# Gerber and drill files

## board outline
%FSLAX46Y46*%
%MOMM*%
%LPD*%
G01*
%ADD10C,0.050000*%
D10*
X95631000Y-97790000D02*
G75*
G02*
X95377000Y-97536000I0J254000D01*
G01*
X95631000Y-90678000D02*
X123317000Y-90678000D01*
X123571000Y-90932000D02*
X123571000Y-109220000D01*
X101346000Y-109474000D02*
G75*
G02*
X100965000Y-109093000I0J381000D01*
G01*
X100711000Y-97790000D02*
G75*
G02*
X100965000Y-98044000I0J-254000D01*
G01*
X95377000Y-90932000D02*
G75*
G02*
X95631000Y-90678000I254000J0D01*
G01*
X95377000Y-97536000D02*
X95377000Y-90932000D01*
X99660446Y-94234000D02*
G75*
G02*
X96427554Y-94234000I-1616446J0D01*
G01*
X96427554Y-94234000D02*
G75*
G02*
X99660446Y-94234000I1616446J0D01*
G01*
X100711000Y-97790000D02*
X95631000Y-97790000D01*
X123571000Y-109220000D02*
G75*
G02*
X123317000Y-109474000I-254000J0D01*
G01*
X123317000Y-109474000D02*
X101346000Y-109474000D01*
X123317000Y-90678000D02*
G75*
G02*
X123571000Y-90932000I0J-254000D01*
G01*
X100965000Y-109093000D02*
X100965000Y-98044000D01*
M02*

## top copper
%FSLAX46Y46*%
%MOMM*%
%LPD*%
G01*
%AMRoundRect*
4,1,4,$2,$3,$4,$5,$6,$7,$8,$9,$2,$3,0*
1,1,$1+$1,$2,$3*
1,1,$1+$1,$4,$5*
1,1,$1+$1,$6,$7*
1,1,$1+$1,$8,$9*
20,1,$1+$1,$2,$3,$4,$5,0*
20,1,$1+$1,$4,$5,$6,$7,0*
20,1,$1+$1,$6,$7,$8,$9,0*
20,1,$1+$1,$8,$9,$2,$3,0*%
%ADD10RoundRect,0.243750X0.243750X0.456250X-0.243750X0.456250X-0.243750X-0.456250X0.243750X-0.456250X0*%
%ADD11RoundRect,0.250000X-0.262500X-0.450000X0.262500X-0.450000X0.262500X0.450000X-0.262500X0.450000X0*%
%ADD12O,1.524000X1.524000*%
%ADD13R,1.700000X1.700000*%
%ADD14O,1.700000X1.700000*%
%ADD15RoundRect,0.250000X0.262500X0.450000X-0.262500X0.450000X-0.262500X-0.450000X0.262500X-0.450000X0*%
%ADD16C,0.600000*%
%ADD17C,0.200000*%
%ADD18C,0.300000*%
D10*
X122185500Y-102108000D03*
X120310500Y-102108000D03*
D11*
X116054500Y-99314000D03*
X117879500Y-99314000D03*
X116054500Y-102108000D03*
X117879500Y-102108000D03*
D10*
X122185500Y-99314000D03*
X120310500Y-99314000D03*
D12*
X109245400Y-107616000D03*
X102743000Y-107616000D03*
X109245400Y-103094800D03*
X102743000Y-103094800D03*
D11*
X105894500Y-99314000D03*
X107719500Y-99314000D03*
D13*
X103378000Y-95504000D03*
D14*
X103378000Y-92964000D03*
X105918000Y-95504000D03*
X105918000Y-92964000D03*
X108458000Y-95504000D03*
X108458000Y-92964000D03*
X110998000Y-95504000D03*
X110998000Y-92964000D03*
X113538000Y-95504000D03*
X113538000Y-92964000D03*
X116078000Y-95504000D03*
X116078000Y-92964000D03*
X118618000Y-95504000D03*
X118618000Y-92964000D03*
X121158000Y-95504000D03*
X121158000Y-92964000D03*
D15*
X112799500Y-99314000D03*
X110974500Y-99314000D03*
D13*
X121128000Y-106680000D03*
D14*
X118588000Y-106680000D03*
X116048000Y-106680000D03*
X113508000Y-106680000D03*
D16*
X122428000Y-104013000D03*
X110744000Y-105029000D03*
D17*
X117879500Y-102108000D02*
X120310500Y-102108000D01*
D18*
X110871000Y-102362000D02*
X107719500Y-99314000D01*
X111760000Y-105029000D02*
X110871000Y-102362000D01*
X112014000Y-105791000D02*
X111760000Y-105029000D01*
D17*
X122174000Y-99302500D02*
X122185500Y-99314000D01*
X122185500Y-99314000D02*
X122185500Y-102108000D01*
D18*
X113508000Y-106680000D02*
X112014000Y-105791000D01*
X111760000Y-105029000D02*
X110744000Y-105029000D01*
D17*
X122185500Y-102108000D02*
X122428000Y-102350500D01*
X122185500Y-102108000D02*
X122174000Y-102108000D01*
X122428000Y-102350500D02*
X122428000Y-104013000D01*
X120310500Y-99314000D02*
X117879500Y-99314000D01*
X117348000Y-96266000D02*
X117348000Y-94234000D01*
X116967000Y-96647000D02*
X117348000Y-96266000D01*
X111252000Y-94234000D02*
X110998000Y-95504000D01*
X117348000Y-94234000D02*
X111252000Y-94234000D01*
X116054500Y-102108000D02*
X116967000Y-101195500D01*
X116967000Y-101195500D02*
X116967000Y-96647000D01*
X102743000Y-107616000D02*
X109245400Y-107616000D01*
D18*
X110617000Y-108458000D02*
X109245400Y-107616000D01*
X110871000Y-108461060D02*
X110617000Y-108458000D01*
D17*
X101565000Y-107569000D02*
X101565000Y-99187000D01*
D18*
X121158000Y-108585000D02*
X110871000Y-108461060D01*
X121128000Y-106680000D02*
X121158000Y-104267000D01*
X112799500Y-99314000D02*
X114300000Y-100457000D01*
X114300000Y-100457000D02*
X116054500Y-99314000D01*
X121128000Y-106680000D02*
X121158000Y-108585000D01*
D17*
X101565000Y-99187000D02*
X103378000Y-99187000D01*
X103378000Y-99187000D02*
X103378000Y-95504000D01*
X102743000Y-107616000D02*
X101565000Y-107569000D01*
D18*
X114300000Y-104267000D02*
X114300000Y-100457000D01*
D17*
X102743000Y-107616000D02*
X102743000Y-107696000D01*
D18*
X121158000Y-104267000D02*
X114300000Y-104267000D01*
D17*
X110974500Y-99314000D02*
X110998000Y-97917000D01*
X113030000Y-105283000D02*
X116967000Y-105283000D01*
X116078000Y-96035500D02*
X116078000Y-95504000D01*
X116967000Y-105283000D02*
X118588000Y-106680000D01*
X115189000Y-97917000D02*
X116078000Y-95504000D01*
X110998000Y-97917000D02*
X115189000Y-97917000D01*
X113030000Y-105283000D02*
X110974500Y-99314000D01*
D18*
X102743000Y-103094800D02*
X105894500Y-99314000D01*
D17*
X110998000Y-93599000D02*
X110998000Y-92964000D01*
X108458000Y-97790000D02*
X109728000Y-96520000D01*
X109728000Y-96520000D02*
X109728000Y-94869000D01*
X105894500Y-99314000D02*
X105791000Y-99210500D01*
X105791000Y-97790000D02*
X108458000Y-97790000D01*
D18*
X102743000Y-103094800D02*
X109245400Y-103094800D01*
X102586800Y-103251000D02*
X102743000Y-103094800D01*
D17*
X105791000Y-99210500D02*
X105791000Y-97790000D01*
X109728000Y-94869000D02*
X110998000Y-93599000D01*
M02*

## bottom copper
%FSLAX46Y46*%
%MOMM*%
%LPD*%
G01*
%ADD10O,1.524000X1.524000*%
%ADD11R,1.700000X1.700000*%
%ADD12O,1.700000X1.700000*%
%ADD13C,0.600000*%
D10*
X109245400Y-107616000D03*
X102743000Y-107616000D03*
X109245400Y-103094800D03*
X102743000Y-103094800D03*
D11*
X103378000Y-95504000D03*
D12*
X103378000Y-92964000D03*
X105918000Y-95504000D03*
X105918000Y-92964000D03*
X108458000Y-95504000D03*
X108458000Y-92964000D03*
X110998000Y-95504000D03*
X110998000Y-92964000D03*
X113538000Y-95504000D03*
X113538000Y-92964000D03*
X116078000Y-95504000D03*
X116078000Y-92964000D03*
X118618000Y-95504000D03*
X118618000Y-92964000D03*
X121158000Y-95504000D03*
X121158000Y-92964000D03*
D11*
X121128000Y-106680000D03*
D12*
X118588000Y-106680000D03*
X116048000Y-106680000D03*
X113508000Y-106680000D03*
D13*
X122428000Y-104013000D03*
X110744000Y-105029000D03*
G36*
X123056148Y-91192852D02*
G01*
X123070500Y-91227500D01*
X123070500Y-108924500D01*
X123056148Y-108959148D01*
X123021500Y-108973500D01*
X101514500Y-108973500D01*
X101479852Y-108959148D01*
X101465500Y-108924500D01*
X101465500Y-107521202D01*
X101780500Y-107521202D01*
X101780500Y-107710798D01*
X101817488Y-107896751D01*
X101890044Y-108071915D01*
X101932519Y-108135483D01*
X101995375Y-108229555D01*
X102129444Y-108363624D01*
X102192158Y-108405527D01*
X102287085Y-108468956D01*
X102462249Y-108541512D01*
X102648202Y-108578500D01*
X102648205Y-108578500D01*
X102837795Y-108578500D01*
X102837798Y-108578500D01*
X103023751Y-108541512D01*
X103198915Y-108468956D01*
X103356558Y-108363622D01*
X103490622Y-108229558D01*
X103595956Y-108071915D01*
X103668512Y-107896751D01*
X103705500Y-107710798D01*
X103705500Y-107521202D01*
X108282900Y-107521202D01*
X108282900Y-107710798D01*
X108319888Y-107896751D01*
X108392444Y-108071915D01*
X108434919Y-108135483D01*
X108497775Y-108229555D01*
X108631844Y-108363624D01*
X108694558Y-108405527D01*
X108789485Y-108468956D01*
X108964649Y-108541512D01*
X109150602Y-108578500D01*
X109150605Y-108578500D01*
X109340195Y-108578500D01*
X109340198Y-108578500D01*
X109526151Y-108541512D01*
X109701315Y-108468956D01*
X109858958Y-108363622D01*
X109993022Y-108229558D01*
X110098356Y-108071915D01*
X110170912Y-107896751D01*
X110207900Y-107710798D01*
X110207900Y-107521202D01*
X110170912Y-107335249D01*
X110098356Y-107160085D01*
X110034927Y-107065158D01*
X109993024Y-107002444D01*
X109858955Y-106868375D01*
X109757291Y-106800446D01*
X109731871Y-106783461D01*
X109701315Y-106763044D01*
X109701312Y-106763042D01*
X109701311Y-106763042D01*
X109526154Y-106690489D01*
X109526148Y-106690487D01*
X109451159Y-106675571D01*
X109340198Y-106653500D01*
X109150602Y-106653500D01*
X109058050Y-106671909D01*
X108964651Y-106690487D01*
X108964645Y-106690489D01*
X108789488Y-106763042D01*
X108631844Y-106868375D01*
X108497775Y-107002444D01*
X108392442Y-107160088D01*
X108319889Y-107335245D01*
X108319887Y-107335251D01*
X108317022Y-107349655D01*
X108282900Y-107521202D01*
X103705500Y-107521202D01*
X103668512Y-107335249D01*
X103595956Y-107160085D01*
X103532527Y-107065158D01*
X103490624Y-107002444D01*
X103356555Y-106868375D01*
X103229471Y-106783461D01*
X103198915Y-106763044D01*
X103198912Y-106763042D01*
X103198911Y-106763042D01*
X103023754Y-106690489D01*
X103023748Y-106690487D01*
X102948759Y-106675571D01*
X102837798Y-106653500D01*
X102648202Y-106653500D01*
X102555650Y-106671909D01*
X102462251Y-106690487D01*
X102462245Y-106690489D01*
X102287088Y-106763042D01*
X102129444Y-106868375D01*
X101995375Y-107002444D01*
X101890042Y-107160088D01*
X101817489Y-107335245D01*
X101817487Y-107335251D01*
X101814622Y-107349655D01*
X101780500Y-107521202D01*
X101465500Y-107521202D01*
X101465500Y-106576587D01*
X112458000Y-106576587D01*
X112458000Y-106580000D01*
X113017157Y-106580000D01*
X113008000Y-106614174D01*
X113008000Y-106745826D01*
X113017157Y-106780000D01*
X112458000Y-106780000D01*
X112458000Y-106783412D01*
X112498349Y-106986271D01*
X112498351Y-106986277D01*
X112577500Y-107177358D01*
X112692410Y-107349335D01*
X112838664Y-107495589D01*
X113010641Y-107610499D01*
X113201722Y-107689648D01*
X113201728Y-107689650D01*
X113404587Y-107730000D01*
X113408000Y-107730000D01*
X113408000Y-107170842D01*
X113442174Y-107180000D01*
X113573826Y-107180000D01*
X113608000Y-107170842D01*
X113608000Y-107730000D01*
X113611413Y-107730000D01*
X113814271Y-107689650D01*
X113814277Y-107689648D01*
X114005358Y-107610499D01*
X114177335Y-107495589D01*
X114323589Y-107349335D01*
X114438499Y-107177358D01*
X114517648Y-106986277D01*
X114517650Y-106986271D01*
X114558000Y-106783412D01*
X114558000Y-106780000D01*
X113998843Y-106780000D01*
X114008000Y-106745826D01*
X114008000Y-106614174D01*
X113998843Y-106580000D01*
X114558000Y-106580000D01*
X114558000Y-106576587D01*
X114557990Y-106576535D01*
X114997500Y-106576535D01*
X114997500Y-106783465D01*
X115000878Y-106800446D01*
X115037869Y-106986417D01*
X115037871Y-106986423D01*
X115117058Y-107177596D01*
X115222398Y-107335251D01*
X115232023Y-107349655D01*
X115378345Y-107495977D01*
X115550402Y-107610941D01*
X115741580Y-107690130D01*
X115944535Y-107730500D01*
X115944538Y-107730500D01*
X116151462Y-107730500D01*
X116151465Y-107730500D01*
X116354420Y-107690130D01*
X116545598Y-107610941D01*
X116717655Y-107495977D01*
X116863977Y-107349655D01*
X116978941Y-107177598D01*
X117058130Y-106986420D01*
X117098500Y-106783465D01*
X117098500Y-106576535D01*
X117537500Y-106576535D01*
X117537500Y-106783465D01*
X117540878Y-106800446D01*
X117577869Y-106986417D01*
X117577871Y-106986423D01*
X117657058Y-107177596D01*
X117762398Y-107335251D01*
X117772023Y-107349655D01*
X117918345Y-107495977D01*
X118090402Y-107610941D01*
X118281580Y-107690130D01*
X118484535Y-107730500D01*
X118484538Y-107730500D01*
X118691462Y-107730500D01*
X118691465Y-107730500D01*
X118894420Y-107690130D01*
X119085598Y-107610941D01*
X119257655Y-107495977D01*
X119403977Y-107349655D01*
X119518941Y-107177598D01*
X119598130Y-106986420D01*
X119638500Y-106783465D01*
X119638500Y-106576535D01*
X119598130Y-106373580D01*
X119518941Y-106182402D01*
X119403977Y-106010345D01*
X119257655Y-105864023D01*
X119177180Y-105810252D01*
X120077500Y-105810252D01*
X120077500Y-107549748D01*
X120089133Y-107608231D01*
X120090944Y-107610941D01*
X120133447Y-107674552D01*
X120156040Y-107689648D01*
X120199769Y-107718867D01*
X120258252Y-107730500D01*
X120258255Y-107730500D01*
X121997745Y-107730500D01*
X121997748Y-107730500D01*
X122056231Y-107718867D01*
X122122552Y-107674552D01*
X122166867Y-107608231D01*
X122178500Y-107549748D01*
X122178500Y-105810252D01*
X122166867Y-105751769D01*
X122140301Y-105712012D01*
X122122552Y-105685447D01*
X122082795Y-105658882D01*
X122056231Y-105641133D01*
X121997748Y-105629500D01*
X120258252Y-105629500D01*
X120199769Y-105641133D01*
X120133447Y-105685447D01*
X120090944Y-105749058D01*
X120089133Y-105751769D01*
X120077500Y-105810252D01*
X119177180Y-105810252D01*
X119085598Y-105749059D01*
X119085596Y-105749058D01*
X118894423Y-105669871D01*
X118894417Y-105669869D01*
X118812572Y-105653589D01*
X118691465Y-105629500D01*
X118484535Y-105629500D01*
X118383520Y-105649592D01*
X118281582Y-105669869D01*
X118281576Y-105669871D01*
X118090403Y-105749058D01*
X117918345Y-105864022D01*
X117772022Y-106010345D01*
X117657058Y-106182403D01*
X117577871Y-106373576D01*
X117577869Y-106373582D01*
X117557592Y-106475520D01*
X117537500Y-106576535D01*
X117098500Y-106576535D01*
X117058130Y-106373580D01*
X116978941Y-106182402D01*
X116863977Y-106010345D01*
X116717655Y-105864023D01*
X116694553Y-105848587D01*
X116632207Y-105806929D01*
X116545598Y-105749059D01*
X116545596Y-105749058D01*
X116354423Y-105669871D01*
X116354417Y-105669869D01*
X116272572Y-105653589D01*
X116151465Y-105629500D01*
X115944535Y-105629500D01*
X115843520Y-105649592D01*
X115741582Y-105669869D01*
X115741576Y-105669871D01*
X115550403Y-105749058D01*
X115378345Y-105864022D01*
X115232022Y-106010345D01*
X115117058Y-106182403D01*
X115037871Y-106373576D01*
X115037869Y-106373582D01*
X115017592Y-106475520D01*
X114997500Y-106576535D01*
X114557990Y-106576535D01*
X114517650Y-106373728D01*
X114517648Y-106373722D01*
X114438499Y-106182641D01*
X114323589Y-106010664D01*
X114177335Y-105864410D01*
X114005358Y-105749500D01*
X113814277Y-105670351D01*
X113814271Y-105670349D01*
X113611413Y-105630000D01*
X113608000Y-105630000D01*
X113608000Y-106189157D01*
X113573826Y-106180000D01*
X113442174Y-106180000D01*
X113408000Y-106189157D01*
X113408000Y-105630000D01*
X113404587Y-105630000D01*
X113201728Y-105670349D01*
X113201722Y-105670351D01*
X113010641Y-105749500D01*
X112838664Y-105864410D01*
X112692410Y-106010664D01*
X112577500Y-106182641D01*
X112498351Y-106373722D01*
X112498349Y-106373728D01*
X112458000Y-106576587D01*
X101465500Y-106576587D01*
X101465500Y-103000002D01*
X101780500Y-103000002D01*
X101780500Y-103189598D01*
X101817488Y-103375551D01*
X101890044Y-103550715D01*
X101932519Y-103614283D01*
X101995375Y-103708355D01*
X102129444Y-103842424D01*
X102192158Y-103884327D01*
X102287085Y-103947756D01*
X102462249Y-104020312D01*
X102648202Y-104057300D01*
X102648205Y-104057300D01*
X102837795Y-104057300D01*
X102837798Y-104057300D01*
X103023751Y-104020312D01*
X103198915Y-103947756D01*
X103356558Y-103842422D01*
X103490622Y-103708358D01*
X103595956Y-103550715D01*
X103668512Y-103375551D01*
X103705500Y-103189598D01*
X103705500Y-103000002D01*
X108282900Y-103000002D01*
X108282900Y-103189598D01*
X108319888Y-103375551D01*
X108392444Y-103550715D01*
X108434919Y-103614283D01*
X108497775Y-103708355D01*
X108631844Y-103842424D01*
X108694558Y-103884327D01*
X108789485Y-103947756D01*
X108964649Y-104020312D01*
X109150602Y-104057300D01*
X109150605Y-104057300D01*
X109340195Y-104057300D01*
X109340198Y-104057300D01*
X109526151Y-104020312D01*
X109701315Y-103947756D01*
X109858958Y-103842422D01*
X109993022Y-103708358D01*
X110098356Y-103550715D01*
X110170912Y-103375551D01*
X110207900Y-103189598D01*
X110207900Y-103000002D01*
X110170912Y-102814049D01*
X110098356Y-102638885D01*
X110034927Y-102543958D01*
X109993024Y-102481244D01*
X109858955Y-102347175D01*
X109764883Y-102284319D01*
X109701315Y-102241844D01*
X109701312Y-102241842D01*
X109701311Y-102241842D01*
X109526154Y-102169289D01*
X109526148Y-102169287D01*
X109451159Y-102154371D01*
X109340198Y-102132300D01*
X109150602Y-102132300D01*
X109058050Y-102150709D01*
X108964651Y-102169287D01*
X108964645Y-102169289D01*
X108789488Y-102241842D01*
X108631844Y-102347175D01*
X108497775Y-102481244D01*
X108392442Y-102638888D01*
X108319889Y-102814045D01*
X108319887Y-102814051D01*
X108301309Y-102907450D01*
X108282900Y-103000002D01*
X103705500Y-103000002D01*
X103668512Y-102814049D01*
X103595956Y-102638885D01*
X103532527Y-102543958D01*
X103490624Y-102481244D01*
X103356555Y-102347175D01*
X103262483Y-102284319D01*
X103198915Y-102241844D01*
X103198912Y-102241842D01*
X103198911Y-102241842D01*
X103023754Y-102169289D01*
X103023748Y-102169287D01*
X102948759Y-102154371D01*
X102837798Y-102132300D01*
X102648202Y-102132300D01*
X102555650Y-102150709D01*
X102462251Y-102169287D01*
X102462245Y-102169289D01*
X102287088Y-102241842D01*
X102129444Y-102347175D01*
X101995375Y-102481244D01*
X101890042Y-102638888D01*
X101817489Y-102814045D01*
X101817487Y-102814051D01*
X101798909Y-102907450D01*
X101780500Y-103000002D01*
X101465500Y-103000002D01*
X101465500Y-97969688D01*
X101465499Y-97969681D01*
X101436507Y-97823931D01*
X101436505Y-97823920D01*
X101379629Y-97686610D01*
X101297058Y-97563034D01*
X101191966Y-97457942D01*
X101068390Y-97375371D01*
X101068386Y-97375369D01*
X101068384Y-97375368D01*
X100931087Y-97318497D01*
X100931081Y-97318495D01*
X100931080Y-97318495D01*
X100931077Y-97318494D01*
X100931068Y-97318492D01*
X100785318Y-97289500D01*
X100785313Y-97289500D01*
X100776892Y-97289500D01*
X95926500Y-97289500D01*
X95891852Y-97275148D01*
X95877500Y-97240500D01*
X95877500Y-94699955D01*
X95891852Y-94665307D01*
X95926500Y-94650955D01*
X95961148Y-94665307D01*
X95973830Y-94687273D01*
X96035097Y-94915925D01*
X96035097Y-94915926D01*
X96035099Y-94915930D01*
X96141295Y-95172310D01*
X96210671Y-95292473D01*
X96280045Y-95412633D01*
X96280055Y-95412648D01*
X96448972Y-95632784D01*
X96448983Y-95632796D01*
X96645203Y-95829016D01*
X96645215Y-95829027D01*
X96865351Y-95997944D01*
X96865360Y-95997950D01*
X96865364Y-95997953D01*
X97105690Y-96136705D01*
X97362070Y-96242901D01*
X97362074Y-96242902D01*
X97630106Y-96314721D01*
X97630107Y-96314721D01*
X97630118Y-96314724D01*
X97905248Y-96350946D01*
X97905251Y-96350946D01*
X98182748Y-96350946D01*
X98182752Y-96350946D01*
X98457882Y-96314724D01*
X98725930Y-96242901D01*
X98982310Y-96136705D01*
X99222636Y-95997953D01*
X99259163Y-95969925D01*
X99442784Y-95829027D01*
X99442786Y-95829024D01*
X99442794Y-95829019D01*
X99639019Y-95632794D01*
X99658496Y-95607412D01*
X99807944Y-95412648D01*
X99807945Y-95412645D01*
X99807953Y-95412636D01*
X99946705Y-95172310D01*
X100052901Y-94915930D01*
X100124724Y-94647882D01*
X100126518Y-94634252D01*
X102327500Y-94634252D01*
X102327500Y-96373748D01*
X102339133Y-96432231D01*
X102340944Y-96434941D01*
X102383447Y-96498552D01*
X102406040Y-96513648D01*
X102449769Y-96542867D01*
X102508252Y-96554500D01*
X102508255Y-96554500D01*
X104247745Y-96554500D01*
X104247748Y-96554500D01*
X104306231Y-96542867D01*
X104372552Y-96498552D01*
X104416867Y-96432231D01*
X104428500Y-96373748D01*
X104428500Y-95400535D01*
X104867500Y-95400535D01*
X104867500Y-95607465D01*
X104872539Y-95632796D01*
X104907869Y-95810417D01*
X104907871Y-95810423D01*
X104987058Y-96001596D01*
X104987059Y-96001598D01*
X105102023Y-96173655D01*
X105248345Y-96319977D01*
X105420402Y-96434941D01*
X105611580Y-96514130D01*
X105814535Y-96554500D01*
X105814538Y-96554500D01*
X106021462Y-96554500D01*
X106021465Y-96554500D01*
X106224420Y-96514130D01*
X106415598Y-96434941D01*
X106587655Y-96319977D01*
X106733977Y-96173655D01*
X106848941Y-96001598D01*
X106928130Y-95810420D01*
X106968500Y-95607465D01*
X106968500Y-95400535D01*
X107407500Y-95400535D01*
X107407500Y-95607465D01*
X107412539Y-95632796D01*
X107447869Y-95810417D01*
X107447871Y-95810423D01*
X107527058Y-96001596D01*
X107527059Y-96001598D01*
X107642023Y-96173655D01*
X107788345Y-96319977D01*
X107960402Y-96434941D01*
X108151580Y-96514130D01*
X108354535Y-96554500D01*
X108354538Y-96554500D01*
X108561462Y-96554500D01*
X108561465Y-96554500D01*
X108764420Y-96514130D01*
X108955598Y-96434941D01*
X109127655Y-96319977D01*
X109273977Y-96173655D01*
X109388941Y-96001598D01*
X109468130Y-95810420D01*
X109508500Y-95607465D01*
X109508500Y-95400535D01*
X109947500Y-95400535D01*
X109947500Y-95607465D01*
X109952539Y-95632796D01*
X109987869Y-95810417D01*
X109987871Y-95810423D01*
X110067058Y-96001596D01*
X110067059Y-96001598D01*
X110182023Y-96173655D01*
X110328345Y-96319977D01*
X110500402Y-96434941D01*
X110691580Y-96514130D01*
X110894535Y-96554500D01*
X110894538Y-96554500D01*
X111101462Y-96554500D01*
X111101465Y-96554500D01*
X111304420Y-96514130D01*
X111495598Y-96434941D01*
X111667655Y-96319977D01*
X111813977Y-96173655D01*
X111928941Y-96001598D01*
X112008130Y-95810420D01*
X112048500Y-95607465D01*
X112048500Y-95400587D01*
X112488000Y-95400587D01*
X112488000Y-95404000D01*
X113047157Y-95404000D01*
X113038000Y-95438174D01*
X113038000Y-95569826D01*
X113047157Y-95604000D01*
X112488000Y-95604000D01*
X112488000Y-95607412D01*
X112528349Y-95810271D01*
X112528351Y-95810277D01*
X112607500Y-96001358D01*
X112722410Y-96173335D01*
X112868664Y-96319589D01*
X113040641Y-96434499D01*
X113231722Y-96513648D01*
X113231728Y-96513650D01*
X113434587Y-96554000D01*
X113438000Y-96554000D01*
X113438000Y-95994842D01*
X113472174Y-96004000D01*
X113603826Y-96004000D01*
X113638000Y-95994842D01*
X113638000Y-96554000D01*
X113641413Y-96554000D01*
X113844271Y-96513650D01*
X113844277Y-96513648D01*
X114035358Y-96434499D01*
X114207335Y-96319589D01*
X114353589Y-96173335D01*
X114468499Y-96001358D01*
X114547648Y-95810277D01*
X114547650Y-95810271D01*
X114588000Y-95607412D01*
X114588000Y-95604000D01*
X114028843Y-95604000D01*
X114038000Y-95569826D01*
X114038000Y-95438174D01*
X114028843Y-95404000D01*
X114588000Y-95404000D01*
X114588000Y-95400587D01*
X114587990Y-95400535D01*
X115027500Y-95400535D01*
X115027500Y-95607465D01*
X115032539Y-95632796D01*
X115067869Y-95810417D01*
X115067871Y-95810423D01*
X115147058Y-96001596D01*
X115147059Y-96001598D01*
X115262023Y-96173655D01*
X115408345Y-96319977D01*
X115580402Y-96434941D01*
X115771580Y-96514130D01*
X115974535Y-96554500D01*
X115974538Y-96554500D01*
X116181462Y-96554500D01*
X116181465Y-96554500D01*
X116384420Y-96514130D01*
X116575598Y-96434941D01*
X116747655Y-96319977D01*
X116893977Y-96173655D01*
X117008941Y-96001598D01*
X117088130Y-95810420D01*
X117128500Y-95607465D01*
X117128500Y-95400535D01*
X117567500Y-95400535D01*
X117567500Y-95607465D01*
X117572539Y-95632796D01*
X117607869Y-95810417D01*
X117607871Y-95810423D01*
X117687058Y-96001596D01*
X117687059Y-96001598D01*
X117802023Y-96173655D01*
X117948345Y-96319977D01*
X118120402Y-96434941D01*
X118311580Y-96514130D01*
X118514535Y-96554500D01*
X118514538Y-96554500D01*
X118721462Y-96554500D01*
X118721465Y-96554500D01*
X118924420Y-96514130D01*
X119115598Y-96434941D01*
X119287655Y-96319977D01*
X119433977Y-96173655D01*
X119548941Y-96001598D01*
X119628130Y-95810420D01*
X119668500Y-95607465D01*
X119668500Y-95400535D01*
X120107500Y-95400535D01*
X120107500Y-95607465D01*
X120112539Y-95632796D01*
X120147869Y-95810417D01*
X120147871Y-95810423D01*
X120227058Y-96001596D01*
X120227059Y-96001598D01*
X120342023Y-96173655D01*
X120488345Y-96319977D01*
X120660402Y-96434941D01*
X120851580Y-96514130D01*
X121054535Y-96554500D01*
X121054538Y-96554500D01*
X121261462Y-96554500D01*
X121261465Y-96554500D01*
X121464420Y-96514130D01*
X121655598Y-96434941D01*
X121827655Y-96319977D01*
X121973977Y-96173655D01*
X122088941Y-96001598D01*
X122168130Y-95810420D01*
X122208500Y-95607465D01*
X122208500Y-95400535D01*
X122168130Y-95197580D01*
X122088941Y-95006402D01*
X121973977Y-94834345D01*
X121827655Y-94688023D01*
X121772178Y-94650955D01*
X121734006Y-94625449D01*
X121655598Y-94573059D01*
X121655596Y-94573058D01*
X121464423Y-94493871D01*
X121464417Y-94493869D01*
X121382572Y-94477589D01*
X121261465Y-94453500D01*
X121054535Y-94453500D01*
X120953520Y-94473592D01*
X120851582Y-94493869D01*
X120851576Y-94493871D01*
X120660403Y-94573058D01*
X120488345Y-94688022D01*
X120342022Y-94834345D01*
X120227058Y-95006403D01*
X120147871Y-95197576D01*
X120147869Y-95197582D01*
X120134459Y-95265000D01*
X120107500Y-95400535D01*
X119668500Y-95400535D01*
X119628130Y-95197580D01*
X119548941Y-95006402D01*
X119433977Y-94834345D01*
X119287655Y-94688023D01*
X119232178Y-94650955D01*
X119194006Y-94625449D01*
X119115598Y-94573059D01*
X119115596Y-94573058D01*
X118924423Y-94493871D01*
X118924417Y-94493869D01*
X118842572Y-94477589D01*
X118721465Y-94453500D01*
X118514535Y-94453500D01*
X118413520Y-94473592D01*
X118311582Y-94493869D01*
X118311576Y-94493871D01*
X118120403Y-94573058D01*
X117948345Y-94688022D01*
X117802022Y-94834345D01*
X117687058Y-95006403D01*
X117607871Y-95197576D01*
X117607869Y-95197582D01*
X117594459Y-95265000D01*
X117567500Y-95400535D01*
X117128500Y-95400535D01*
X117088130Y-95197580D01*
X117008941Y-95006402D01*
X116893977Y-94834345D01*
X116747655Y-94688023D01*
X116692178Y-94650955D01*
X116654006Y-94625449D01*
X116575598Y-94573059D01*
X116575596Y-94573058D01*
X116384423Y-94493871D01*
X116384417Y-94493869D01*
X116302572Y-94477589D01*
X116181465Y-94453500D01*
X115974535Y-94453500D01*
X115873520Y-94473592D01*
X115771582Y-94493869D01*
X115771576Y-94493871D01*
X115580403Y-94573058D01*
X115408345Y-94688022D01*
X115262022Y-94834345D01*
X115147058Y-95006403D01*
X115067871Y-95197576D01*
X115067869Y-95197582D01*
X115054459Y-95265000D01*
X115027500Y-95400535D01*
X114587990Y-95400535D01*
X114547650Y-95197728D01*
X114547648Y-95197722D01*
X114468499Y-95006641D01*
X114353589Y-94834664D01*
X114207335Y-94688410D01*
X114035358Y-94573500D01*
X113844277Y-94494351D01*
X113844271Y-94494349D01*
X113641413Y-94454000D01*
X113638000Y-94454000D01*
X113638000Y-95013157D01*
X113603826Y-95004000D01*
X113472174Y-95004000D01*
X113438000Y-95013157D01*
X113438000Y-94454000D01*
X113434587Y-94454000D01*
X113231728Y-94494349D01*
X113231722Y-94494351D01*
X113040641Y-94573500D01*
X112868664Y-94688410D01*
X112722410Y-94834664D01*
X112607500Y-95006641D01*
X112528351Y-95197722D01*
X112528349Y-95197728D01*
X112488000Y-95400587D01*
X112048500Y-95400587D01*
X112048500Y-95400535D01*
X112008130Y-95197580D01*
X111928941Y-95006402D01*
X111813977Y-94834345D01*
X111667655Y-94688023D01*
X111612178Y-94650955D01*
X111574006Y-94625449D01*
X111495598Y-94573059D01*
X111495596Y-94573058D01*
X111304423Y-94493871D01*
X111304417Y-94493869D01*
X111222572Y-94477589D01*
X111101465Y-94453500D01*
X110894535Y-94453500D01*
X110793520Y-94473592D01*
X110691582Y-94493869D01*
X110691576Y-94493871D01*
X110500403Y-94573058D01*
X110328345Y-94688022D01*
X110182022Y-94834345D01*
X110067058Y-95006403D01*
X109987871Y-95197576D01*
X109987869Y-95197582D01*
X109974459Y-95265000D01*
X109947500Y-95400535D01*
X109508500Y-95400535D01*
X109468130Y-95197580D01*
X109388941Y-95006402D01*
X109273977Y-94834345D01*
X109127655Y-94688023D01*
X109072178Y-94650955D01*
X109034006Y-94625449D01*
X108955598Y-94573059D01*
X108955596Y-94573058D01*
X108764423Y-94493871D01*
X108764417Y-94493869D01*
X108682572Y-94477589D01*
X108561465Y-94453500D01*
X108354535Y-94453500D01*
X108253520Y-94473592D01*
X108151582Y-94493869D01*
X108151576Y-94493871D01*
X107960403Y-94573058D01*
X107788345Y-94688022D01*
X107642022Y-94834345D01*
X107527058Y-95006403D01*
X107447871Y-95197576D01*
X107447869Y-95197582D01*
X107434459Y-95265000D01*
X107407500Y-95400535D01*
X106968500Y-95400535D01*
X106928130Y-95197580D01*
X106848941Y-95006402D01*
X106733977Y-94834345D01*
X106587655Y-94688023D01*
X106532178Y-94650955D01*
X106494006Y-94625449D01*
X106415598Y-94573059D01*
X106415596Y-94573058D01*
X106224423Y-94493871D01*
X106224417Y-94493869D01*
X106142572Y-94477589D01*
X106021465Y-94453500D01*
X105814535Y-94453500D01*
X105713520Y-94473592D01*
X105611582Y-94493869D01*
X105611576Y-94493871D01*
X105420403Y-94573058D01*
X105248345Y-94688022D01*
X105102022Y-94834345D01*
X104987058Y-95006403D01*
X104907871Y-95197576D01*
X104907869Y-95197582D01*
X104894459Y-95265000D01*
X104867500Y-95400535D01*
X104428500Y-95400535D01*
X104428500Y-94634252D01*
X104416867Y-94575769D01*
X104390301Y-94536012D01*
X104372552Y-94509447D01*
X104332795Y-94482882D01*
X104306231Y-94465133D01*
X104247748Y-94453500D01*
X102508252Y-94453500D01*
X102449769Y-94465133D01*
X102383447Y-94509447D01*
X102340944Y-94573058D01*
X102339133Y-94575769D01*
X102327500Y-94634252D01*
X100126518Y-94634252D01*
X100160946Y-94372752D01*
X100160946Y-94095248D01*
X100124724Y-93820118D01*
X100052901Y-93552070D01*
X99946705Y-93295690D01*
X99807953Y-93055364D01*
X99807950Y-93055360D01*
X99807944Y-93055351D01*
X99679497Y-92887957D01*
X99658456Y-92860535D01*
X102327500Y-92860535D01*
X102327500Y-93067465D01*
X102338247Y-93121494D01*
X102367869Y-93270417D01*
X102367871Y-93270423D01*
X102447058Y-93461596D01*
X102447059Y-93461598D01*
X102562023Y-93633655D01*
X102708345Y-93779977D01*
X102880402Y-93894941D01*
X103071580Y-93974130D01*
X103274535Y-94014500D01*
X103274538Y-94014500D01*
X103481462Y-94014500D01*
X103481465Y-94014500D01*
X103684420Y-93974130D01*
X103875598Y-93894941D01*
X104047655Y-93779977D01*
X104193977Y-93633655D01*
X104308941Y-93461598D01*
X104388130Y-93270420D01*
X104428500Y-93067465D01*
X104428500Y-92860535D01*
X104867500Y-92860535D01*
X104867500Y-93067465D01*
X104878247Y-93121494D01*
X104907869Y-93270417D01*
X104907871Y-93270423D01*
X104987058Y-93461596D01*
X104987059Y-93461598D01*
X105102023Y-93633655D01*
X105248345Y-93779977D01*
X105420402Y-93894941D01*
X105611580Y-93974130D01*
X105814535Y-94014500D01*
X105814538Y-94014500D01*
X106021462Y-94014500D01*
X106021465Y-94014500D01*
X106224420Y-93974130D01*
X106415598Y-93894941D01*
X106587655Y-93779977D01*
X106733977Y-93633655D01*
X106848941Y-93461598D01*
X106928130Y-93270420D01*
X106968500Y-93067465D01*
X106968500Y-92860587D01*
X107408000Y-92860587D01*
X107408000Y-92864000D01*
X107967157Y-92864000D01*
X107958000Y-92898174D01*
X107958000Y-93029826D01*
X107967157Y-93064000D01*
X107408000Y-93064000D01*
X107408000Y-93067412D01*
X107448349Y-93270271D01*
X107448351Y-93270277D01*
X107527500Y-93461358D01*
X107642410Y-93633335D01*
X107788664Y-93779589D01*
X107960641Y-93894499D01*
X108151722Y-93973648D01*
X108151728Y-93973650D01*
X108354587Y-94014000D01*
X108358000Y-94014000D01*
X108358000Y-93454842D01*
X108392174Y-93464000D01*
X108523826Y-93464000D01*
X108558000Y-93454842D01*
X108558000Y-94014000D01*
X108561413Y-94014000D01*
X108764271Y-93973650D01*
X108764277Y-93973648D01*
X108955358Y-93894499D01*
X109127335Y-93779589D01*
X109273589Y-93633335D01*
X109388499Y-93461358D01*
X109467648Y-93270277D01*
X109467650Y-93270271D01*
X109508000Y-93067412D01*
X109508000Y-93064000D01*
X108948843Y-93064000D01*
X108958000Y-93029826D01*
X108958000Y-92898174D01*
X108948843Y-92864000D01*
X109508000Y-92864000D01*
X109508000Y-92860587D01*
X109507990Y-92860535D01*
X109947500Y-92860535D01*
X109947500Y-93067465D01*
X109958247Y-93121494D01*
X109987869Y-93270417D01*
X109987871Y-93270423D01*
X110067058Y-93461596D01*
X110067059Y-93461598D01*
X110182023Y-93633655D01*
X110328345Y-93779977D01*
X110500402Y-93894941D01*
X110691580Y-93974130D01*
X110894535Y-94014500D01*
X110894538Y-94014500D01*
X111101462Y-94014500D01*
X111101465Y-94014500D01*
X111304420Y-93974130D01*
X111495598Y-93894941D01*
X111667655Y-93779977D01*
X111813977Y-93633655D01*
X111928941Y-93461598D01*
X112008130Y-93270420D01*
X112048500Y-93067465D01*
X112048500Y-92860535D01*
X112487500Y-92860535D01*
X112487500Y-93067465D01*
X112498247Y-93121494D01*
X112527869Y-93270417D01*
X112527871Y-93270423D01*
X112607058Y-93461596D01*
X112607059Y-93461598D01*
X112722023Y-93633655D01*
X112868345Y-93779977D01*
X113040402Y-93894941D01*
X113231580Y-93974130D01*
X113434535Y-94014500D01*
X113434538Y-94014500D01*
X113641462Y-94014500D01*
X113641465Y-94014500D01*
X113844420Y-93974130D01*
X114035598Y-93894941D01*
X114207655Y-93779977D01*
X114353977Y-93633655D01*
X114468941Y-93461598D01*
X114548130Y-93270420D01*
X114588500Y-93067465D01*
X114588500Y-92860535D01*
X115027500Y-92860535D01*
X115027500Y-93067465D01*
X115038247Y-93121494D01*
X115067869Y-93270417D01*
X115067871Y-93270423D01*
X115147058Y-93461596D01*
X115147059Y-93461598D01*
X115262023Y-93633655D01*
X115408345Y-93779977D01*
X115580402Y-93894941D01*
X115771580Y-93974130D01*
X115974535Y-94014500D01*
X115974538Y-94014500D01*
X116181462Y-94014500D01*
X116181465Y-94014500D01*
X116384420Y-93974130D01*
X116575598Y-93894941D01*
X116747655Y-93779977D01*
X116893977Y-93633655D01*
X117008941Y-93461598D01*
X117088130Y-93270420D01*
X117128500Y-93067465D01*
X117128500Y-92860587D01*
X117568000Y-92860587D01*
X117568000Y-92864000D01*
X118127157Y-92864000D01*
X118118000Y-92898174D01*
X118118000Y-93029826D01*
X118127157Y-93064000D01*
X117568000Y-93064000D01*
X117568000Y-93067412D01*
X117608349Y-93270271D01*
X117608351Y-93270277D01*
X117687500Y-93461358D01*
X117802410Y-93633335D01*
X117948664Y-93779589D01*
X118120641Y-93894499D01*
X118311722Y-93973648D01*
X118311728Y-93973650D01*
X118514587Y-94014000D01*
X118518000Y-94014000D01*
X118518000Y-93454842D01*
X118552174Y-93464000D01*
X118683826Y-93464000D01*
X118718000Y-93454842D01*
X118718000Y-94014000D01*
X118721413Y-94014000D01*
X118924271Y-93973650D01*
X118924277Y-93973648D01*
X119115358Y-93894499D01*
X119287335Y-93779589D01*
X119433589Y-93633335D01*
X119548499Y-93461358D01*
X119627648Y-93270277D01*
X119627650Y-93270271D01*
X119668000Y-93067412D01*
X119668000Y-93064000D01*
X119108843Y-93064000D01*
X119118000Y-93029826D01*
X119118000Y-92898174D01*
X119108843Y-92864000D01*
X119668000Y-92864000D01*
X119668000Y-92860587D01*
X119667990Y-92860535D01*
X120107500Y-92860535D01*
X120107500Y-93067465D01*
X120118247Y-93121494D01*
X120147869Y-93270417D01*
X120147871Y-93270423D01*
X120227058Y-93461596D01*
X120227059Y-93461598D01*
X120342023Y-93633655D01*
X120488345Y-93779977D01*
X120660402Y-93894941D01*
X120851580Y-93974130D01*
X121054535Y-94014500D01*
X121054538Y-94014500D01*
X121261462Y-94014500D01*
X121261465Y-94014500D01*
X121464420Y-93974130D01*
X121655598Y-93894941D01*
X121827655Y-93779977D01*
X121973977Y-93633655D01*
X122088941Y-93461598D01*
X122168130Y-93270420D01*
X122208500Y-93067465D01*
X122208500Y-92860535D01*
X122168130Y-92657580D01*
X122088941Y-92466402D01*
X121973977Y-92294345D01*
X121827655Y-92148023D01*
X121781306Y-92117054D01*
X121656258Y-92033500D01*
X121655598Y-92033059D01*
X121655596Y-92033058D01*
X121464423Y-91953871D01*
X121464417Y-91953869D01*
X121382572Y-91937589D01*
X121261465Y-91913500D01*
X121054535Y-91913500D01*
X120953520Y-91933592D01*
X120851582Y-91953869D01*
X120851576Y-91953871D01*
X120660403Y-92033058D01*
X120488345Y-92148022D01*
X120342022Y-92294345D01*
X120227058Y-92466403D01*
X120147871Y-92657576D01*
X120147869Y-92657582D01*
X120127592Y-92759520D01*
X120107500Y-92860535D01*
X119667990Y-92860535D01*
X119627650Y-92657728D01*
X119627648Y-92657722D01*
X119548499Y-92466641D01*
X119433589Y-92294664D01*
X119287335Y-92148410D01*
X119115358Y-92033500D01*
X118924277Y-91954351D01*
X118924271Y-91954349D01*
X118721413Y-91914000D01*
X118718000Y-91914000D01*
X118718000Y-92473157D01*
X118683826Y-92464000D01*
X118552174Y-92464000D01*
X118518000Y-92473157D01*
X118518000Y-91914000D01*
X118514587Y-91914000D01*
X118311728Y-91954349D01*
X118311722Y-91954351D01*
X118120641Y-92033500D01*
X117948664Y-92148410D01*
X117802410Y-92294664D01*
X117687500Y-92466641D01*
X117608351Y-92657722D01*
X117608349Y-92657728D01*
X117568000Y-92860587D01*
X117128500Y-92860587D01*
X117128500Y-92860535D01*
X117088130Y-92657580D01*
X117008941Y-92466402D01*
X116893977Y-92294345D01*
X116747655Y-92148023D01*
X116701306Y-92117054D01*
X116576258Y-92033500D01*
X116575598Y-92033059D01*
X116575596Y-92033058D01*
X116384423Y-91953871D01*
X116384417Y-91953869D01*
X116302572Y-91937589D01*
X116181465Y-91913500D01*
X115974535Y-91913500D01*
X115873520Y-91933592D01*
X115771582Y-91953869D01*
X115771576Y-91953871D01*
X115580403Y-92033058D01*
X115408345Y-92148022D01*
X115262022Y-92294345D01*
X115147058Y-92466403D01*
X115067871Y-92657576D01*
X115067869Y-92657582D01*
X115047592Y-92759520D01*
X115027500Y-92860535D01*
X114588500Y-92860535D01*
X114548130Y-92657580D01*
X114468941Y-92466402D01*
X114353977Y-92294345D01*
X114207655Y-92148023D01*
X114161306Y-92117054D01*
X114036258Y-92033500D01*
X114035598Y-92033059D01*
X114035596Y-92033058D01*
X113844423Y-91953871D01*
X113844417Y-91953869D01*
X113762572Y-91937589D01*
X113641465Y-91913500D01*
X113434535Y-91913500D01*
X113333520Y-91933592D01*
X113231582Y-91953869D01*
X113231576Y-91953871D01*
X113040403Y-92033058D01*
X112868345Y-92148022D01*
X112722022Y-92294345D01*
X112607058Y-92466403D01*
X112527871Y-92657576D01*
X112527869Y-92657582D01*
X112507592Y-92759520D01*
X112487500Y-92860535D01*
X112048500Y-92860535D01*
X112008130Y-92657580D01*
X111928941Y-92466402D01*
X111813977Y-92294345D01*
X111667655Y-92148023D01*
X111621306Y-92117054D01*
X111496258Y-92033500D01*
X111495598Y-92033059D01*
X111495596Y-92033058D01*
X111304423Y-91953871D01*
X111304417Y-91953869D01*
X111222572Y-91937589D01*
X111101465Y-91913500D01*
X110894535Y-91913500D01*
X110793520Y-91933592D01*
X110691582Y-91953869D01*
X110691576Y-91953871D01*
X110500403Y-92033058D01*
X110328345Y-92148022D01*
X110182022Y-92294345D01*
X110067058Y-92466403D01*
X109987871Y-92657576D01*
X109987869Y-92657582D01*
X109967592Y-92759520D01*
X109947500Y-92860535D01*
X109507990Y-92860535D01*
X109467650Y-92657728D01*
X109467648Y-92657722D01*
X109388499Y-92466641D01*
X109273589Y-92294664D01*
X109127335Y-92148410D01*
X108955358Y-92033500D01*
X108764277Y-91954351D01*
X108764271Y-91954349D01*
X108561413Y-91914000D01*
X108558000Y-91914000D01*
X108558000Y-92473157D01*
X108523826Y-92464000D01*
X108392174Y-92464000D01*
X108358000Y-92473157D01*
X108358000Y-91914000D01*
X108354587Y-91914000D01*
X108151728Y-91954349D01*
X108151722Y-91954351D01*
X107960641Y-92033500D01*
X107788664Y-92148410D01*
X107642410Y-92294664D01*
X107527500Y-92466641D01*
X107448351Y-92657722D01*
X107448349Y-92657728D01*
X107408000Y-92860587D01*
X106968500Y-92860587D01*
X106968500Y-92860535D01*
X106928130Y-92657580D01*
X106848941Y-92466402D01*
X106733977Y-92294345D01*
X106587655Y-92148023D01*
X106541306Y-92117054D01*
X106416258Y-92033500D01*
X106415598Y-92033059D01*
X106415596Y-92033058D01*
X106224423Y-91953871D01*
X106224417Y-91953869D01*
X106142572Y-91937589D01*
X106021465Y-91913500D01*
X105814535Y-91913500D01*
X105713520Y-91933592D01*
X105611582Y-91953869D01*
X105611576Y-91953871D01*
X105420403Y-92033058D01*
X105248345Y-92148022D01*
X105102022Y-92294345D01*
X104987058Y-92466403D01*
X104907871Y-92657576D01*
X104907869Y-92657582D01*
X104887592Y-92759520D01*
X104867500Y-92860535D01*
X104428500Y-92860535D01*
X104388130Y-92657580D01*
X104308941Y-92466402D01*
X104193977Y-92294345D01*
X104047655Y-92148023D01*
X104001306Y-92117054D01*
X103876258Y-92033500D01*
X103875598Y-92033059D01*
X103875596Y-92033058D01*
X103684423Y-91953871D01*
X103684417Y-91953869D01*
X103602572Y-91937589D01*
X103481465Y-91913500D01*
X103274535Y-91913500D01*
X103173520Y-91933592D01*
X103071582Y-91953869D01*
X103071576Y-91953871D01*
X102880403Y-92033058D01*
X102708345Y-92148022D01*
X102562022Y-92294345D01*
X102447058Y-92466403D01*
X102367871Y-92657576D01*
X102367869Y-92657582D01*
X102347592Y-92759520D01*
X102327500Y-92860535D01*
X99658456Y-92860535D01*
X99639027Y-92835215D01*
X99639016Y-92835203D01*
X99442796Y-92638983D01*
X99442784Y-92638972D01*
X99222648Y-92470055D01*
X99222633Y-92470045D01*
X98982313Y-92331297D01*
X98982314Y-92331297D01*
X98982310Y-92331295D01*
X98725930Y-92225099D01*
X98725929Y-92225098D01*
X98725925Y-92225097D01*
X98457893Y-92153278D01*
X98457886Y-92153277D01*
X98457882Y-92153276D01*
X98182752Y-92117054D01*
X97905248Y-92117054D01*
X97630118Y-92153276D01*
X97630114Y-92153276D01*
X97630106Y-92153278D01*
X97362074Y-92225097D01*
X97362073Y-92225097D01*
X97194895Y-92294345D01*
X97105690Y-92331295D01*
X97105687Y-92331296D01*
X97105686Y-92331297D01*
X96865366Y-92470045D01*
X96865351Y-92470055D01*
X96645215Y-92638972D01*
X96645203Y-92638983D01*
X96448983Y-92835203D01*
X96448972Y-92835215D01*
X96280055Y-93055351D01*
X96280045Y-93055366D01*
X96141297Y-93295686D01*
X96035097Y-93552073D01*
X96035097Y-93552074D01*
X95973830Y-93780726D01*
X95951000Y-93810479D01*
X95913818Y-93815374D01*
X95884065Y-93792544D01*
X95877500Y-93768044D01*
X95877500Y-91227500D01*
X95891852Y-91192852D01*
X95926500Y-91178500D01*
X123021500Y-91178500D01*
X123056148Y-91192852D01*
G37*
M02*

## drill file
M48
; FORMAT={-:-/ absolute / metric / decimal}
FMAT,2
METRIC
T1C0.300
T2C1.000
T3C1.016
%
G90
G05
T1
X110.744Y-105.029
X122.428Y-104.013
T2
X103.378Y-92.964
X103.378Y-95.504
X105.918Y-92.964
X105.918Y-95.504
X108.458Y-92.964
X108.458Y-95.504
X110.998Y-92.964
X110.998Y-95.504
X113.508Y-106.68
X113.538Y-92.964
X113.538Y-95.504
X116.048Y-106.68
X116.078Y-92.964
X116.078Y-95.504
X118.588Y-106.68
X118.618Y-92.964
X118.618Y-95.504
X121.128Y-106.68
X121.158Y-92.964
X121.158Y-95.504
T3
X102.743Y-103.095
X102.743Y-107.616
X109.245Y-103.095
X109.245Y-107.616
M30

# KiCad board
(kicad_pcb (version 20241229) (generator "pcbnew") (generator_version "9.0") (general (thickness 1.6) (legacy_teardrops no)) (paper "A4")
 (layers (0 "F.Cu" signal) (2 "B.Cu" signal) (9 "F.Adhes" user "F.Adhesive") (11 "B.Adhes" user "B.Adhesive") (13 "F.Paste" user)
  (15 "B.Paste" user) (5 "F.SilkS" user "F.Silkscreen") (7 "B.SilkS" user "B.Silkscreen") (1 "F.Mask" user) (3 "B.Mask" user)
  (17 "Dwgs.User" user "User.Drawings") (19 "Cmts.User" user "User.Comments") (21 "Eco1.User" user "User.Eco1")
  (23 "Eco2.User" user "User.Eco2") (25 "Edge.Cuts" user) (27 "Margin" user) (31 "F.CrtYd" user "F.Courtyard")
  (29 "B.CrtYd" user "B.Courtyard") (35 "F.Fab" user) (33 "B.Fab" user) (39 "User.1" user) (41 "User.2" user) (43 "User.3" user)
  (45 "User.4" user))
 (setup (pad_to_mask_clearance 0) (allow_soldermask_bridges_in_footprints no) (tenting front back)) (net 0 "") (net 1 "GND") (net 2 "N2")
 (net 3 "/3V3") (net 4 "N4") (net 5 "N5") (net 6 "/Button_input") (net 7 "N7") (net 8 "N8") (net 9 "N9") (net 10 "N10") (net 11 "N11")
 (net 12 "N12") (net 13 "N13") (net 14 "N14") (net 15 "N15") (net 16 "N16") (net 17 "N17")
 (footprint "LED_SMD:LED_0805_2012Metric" (layer "F.Cu") (at 121.248 102.108 180)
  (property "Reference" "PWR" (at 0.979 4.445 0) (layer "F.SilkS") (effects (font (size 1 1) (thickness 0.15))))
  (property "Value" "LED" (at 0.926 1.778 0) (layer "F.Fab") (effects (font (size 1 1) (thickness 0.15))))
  (pad "1" smd roundrect (at -0.9375 0 180) (size 0.975 1.4) (layers "F.Cu" "F.Mask" "F.Paste") (roundrect_rratio 0.25) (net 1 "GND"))
  (pad "2" smd roundrect (at 0.9375 0 180) (size 0.975 1.4) (layers "F.Cu" "F.Mask" "F.Paste") (roundrect_rratio 0.25) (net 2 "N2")))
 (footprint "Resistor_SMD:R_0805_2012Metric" (layer "F.Cu") (at 116.967 99.314)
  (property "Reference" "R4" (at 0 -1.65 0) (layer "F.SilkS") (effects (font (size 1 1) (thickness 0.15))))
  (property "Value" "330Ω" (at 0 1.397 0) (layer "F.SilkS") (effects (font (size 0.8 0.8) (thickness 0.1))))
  (pad "1" smd roundrect (at -0.9125 0) (size 1.025 1.4) (layers "F.Cu" "F.Mask" "F.Paste") (roundrect_rratio 0.243902) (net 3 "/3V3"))
  (pad "2" smd roundrect (at 0.9125 0) (size 1.025 1.4) (layers "F.Cu" "F.Mask" "F.Paste") (roundrect_rratio 0.243902) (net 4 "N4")))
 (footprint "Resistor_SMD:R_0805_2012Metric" (layer "F.Cu") (at 116.967 102.108)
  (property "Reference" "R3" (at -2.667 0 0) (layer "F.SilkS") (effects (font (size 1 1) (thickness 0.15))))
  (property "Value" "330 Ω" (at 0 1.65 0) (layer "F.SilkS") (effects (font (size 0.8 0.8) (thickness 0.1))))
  (pad "1" smd roundrect (at -0.9125 0) (size 1.025 1.4) (layers "F.Cu" "F.Mask" "F.Paste") (roundrect_rratio 0.243902) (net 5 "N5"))
  (pad "2" smd roundrect (at 0.9125 0) (size 1.025 1.4) (layers "F.Cu" "F.Mask" "F.Paste") (roundrect_rratio 0.243902) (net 2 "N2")))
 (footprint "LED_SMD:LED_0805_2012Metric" (layer "F.Cu") (at 121.248 99.314 180)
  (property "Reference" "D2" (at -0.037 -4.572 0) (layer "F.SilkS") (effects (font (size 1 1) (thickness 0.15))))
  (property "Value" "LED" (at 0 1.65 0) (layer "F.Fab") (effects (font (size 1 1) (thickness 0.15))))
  (pad "1" smd roundrect (at -0.9375 0 180) (size 0.975 1.4) (layers "F.Cu" "F.Mask" "F.Paste") (roundrect_rratio 0.25) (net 1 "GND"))
  (pad "2" smd roundrect (at 0.9375 0 180) (size 0.975 1.4) (layers "F.Cu" "F.Mask" "F.Paste") (roundrect_rratio 0.25) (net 4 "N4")))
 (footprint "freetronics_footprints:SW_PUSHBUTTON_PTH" (layer "F.Cu") (at 105.9942 105.3554 180)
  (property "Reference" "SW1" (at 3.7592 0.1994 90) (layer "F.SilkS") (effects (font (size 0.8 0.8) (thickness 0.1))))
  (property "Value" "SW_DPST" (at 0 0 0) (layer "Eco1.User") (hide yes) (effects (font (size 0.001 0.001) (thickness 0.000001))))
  (pad "1" thru_hole oval (at -3.2512 -2.2606 180) (size 1.524 1.524) (drill 1.016) (layers "*.Cu" "*.Mask") (remove_unused_layers no)
   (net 3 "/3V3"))
  (pad "1" thru_hole oval (at 3.2512 -2.2606 180) (size 1.524 1.524) (drill 1.016) (layers "*.Cu" "*.Mask") (remove_unused_layers no)
   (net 3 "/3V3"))
  (pad "2" thru_hole oval (at -3.2512 2.2606 180) (size 1.524 1.524) (drill 1.016) (layers "*.Cu" "*.Mask") (remove_unused_layers no)
   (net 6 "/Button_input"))
  (pad "2" thru_hole oval (at 3.2512 2.2606 180) (size 1.524 1.524) (drill 1.016) (layers "*.Cu" "*.Mask") (remove_unused_layers no)
   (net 6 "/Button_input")))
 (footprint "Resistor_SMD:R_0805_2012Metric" (layer "F.Cu") (at 106.807 99.314)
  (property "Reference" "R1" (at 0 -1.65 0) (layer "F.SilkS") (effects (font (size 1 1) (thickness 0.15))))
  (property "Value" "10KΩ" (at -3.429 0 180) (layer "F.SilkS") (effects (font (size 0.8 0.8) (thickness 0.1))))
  (pad "1" smd roundrect (at -0.9125 0) (size 1.025 1.4) (layers "F.Cu" "F.Mask" "F.Paste") (roundrect_rratio 0.243902)
   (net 6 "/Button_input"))
  (pad "2" smd roundrect (at 0.9125 0) (size 1.025 1.4) (layers "F.Cu" "F.Mask" "F.Paste") (roundrect_rratio 0.243902) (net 1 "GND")))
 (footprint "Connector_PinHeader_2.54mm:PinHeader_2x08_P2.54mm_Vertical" (layer "F.Cu") (at 103.378 95.504 90)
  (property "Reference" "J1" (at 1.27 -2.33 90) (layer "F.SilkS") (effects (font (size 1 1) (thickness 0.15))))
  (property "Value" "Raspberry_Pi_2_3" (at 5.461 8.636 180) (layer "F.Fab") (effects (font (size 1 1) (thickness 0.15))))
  (pad "1" thru_hole rect (at 0 0 90) (size 1.7 1.7) (drill 1) (layers "*.Cu" "*.Mask") (remove_unused_layers no) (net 3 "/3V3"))
  (pad "2" thru_hole oval (at 2.54 0 90) (size 1.7 1.7) (drill 1) (layers "*.Cu" "*.Mask") (remove_unused_layers no) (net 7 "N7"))
  (pad "3" thru_hole oval (at 0 2.54 90) (size 1.7 1.7) (drill 1) (layers "*.Cu" "*.Mask") (remove_unused_layers no) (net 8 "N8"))
  (pad "4" thru_hole oval (at 2.54 2.54 90) (size 1.7 1.7) (drill 1) (layers "*.Cu" "*.Mask") (remove_unused_layers no) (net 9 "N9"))
  (pad "5" thru_hole oval (at 0 5.08 90) (size 1.7 1.7) (drill 1) (layers "*.Cu" "*.Mask") (remove_unused_layers no) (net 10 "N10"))
  (pad "6" thru_hole oval (at 2.54 5.08 90) (size 1.7 1.7) (drill 1) (layers "*.Cu" "*.Mask") (remove_unused_layers no) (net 1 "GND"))
  (pad "7" thru_hole oval (at 0 7.62 90) (size 1.7 1.7) (drill 1) (layers "*.Cu" "*.Mask") (remove_unused_layers no) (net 5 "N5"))
  (pad "8" thru_hole oval (at 2.54 7.62 90) (size 1.7 1.7) (drill 1) (layers "*.Cu" "*.Mask") (remove_unused_layers no)
   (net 6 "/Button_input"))
  (pad "9" thru_hole oval (at 0 10.16 90) (size 1.7 1.7) (drill 1) (layers "*.Cu" "*.Mask") (remove_unused_layers no) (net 1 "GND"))
  (pad "10" thru_hole oval (at 2.54 10.16 90) (size 1.7 1.7) (drill 1) (layers "*.Cu" "*.Mask") (remove_unused_layers no) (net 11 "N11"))
  (pad "11" thru_hole oval (at 0 12.7 90) (size 1.7 1.7) (drill 1) (layers "*.Cu" "*.Mask") (remove_unused_layers no) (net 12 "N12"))
  (pad "12" thru_hole oval (at 2.54 12.7 90) (size 1.7 1.7) (drill 1) (layers "*.Cu" "*.Mask") (remove_unused_layers no) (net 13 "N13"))
  (pad "13" thru_hole oval (at 0 15.24 90) (size 1.7 1.7) (drill 1) (layers "*.Cu" "*.Mask") (remove_unused_layers no) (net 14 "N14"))
  (pad "14" thru_hole oval (at 2.54 15.24 90) (size 1.7 1.7) (drill 1) (layers "*.Cu" "*.Mask") (remove_unused_layers no) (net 1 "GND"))
  (pad "15" thru_hole oval (at 0 17.78 90) (size 1.7 1.7) (drill 1) (layers "*.Cu" "*.Mask") (remove_unused_layers no) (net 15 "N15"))
  (pad "16" thru_hole oval (at 2.54 17.78 90) (size 1.7 1.7) (drill 1) (layers "*.Cu" "*.Mask") (remove_unused_layers no) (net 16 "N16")))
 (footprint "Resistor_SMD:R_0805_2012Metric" (layer "F.Cu") (at 111.887 99.314 180)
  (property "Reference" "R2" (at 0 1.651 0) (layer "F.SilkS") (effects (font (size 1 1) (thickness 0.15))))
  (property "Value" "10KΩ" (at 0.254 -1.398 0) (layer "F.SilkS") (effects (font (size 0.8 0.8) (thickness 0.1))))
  (pad "1" smd roundrect (at -0.9125 0 180) (size 1.025 1.4) (layers "F.Cu" "F.Mask" "F.Paste") (roundrect_rratio 0.243902) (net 3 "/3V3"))
  (pad "2" smd roundrect (at 0.9125 0 180) (size 1.025 1.4) (layers "F.Cu" "F.Mask" "F.Paste") (roundrect_rratio 0.243902) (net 12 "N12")))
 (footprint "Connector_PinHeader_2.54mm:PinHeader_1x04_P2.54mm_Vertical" (layer "F.Cu") (at 121.128 106.68 -90)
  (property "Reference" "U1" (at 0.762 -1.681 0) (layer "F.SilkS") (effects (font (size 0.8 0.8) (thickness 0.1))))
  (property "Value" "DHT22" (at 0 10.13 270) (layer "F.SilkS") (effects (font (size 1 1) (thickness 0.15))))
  (pad "1" thru_hole rect (at 0 0 270) (size 1.7 1.7) (drill 1) (layers "*.Cu" "*.Mask") (remove_unused_layers no) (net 3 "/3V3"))
  (pad "2" thru_hole oval (at 0 2.54 270) (size 1.7 1.7) (drill 1) (layers "*.Cu" "*.Mask") (remove_unused_layers no) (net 12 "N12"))
  (pad "3" thru_hole oval (at 0 5.08 270) (size 1.7 1.7) (drill 1) (layers "*.Cu" "*.Mask") (remove_unused_layers no) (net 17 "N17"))
  (pad "4" thru_hole oval (at 0 7.62 270) (size 1.7 1.7) (drill 1) (layers "*.Cu" "*.Mask") (remove_unused_layers no) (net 1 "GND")))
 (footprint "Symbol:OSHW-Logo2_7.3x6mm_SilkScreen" (layer "B.Cu") (at 105.41 99.695 180)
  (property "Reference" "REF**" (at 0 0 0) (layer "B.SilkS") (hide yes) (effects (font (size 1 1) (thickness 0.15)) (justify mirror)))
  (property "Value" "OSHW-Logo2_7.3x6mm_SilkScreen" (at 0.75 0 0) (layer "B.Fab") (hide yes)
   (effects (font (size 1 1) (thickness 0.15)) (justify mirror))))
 (gr_arc (start 95.631 97.79) (mid 95.451395 97.715605) (end 95.377 97.536) (stroke (width 0.05) (type default)) (layer "Edge.Cuts"))
 (gr_line (start 95.631 90.678) (end 123.317 90.678) (stroke (width 0.05) (type default)) (layer "Edge.Cuts"))
 (gr_line (start 123.571 90.932) (end 123.571 109.22) (stroke (width 0.05) (type default)) (layer "Edge.Cuts"))
 (gr_arc (start 101.346 109.474) (mid 101.076592 109.362408) (end 100.965 109.093) (stroke (width 0.05) (type default)) (layer "Edge.Cuts"))
 (gr_arc (start 100.711 97.79) (mid 100.890605 97.864395) (end 100.965 98.044) (stroke (width 0.05) (type default)) (layer "Edge.Cuts"))
 (gr_arc (start 95.377 90.932) (mid 95.451395 90.752395) (end 95.631 90.678) (stroke (width 0.05) (type default)) (layer "Edge.Cuts"))
 (gr_line (start 95.377 97.536) (end 95.377 90.932) (stroke (width 0.05) (type default)) (layer "Edge.Cuts"))
 (gr_circle (center 98.044 94.234) (end 99.187 95.377) (stroke (width 0.05) (type default)) (fill no) (layer "Edge.Cuts"))
 (gr_line (start 100.711 97.79) (end 95.631 97.79) (stroke (width 0.05) (type default)) (layer "Edge.Cuts"))
 (gr_arc (start 123.571 109.22) (mid 123.496605 109.399605) (end 123.317 109.474) (stroke (width 0.05) (type default)) (layer "Edge.Cuts"))
 (gr_line (start 123.317 109.474) (end 101.346 109.474) (stroke (width 0.05) (type default)) (layer "Edge.Cuts"))
 (gr_arc (start 123.317 90.678) (mid 123.496605 90.752395) (end 123.571 90.932) (stroke (width 0.05) (type default)) (layer "Edge.Cuts"))
 (gr_line (start 100.965 109.093) (end 100.965 98.044) (stroke (width 0.05) (type default)) (layer "Edge.Cuts"))
 (segment (start 117.8795 102.108) (end 120.3105 102.108) (width 0.2) (layer "F.Cu") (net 2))
 (segment (start 110.871 102.362) (end 107.7195 99.314) (width 0.3) (layer "F.Cu") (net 1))
 (segment (start 111.76 105.029) (end 110.871 102.362) (width 0.3) (layer "F.Cu") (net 1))
 (segment (start 112.014 105.791) (end 111.76 105.029) (width 0.3) (layer "F.Cu") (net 1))
 (segment (start 122.174 99.3025) (end 122.1855 99.314) (width 0.2) (layer "F.Cu") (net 1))
 (segment (start 122.1855 99.314) (end 122.1855 102.108) (width 0.2) (layer "F.Cu") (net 1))
 (segment (start 113.508 106.68) (end 112.014 105.791) (width 0.3) (layer "F.Cu") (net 1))
 (segment (start 111.76 105.029) (end 110.744 105.029) (width 0.3) (layer "F.Cu") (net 1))
 (segment (start 122.1855 102.108) (end 122.428 102.3505) (width 0.2) (layer "F.Cu") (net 1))
 (segment (start 122.1855 102.108) (end 122.174 102.108) (width 0.2) (layer "F.Cu") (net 1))
 (segment (start 122.428 102.3505) (end 122.428 104.013) (width 0.2) (layer "F.Cu") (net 1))
 (via (at 122.428 104.013) (size 0.6) (drill 0.3) (layers "F.Cu" "B.Cu") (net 1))
 (via (at 110.744 105.029) (size 0.6) (drill 0.3) (layers "F.Cu" "B.Cu") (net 1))
 (segment (start 120.3105 99.314) (end 117.8795 99.314) (width 0.2) (layer "F.Cu") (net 4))
 (segment (start 117.348 96.266) (end 117.348 94.234) (width 0.2) (layer "F.Cu") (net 5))
 (segment (start 116.967 96.647) (end 117.348 96.266) (width 0.2) (layer "F.Cu") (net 5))
 (segment (start 111.252 94.234) (end 110.998 95.504) (width 0.2) (layer "F.Cu") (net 5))
 (segment (start 117.348 94.234) (end 111.252 94.234) (width 0.2) (layer "F.Cu") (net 5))
 (segment (start 116.0545 102.108) (end 116.967 101.1955) (width 0.2) (layer "F.Cu") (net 5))
 (segment (start 116.967 101.1955) (end 116.967 96.647) (width 0.2) (layer "F.Cu") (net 5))
 (segment (start 102.743 107.616) (end 109.2454 107.616) (width 0.2) (layer "F.Cu") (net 3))
 (segment (start 110.617 108.458) (end 109.2454 107.616) (width 0.3) (layer "F.Cu") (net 3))
 (segment (start 110.871 108.46106) (end 110.617 108.458) (width 0.3) (layer "F.Cu") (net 3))
 (segment (start 101.565 107.569) (end 101.565 99.187) (width 0.2) (layer "F.Cu") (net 3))
 (segment (start 121.158 108.585) (end 110.871 108.46106) (width 0.3) (layer "F.Cu") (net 3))
 (segment (start 121.128 106.68) (end 121.158 104.267) (width 0.3) (layer "F.Cu") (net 3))
 (segment (start 112.7995 99.314) (end 114.3 100.457) (width 0.3) (layer "F.Cu") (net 3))
 (segment (start 114.3 100.457) (end 116.0545 99.314) (width 0.3) (layer "F.Cu") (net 3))
 (segment (start 121.128 106.68) (end 121.158 108.585) (width 0.3) (layer "F.Cu") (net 3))
 (segment (start 101.565 99.187) (end 103.378 99.187) (width 0.2) (layer "F.Cu") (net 3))
 (segment (start 103.378 99.187) (end 103.378 95.504) (width 0.2) (layer "F.Cu") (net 3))
 (segment (start 102.743 107.616) (end 101.565 107.569) (width 0.2) (layer "F.Cu") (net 3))
 (segment (start 114.3 104.267) (end 114.3 100.457) (width 0.3) (layer "F.Cu") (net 3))
 (segment (start 102.743 107.616) (end 102.743 107.696) (width 0.2) (layer "F.Cu") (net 3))
 (segment (start 121.158 104.267) (end 114.3 104.267) (width 0.3) (layer "F.Cu") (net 3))
 (segment (start 110.9745 99.314) (end 110.998 97.917) (width 0.2) (layer "F.Cu") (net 12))
 (segment (start 113.03 105.283) (end 116.967 105.283) (width 0.2) (layer "F.Cu") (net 12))
 (segment (start 116.078 96.0355) (end 116.078 95.504) (width 0.2) (layer "F.Cu") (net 12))
 (segment (start 116.967 105.283) (end 118.588 106.68) (width 0.2) (layer "F.Cu") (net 12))
 (segment (start 115.189 97.917) (end 116.078 95.504) (width 0.2) (layer "F.Cu") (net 12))
 (segment (start 110.998 97.917) (end 115.189 97.917) (width 0.2) (layer "F.Cu") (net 12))
 (segment (start 113.03 105.283) (end 110.9745 99.314) (width 0.2) (layer "F.Cu") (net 12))
 (segment (start 102.743 103.0948) (end 105.8945 99.314) (width 0.3) (layer "F.Cu") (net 6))
 (segment (start 110.998 93.599) (end 110.998 92.964) (width 0.2) (layer "F.Cu") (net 6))
 (segment (start 108.458 97.79) (end 109.728 96.52) (width 0.2) (layer "F.Cu") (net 6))
 (segment (start 109.728 96.52) (end 109.728 94.869) (width 0.2) (layer "F.Cu") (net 6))
 (segment (start 105.8945 99.314) (end 105.791 99.2105) (width 0.2) (layer "F.Cu") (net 6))
 (segment (start 105.791 97.79) (end 108.458 97.79) (width 0.2) (layer "F.Cu") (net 6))
 (segment (start 102.743 103.0948) (end 109.2454 103.0948) (width 0.3) (layer "F.Cu") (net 6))
 (segment (start 102.5868 103.251) (end 102.743 103.0948) (width 0.3) (layer "F.Cu") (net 6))
 (segment (start 105.791 99.2105) (end 105.791 97.79) (width 0.2) (layer "F.Cu") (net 6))
 (segment (start 109.728 94.869) (end 110.998 93.599) (width 0.2) (layer "F.Cu") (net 6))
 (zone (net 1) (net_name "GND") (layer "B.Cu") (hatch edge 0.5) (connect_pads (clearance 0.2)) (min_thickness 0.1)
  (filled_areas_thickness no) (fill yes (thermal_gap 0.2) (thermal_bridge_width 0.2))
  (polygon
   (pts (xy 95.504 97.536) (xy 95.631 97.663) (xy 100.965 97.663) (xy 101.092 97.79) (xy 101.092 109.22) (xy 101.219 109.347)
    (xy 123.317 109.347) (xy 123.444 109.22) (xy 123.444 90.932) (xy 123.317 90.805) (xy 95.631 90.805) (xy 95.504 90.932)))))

